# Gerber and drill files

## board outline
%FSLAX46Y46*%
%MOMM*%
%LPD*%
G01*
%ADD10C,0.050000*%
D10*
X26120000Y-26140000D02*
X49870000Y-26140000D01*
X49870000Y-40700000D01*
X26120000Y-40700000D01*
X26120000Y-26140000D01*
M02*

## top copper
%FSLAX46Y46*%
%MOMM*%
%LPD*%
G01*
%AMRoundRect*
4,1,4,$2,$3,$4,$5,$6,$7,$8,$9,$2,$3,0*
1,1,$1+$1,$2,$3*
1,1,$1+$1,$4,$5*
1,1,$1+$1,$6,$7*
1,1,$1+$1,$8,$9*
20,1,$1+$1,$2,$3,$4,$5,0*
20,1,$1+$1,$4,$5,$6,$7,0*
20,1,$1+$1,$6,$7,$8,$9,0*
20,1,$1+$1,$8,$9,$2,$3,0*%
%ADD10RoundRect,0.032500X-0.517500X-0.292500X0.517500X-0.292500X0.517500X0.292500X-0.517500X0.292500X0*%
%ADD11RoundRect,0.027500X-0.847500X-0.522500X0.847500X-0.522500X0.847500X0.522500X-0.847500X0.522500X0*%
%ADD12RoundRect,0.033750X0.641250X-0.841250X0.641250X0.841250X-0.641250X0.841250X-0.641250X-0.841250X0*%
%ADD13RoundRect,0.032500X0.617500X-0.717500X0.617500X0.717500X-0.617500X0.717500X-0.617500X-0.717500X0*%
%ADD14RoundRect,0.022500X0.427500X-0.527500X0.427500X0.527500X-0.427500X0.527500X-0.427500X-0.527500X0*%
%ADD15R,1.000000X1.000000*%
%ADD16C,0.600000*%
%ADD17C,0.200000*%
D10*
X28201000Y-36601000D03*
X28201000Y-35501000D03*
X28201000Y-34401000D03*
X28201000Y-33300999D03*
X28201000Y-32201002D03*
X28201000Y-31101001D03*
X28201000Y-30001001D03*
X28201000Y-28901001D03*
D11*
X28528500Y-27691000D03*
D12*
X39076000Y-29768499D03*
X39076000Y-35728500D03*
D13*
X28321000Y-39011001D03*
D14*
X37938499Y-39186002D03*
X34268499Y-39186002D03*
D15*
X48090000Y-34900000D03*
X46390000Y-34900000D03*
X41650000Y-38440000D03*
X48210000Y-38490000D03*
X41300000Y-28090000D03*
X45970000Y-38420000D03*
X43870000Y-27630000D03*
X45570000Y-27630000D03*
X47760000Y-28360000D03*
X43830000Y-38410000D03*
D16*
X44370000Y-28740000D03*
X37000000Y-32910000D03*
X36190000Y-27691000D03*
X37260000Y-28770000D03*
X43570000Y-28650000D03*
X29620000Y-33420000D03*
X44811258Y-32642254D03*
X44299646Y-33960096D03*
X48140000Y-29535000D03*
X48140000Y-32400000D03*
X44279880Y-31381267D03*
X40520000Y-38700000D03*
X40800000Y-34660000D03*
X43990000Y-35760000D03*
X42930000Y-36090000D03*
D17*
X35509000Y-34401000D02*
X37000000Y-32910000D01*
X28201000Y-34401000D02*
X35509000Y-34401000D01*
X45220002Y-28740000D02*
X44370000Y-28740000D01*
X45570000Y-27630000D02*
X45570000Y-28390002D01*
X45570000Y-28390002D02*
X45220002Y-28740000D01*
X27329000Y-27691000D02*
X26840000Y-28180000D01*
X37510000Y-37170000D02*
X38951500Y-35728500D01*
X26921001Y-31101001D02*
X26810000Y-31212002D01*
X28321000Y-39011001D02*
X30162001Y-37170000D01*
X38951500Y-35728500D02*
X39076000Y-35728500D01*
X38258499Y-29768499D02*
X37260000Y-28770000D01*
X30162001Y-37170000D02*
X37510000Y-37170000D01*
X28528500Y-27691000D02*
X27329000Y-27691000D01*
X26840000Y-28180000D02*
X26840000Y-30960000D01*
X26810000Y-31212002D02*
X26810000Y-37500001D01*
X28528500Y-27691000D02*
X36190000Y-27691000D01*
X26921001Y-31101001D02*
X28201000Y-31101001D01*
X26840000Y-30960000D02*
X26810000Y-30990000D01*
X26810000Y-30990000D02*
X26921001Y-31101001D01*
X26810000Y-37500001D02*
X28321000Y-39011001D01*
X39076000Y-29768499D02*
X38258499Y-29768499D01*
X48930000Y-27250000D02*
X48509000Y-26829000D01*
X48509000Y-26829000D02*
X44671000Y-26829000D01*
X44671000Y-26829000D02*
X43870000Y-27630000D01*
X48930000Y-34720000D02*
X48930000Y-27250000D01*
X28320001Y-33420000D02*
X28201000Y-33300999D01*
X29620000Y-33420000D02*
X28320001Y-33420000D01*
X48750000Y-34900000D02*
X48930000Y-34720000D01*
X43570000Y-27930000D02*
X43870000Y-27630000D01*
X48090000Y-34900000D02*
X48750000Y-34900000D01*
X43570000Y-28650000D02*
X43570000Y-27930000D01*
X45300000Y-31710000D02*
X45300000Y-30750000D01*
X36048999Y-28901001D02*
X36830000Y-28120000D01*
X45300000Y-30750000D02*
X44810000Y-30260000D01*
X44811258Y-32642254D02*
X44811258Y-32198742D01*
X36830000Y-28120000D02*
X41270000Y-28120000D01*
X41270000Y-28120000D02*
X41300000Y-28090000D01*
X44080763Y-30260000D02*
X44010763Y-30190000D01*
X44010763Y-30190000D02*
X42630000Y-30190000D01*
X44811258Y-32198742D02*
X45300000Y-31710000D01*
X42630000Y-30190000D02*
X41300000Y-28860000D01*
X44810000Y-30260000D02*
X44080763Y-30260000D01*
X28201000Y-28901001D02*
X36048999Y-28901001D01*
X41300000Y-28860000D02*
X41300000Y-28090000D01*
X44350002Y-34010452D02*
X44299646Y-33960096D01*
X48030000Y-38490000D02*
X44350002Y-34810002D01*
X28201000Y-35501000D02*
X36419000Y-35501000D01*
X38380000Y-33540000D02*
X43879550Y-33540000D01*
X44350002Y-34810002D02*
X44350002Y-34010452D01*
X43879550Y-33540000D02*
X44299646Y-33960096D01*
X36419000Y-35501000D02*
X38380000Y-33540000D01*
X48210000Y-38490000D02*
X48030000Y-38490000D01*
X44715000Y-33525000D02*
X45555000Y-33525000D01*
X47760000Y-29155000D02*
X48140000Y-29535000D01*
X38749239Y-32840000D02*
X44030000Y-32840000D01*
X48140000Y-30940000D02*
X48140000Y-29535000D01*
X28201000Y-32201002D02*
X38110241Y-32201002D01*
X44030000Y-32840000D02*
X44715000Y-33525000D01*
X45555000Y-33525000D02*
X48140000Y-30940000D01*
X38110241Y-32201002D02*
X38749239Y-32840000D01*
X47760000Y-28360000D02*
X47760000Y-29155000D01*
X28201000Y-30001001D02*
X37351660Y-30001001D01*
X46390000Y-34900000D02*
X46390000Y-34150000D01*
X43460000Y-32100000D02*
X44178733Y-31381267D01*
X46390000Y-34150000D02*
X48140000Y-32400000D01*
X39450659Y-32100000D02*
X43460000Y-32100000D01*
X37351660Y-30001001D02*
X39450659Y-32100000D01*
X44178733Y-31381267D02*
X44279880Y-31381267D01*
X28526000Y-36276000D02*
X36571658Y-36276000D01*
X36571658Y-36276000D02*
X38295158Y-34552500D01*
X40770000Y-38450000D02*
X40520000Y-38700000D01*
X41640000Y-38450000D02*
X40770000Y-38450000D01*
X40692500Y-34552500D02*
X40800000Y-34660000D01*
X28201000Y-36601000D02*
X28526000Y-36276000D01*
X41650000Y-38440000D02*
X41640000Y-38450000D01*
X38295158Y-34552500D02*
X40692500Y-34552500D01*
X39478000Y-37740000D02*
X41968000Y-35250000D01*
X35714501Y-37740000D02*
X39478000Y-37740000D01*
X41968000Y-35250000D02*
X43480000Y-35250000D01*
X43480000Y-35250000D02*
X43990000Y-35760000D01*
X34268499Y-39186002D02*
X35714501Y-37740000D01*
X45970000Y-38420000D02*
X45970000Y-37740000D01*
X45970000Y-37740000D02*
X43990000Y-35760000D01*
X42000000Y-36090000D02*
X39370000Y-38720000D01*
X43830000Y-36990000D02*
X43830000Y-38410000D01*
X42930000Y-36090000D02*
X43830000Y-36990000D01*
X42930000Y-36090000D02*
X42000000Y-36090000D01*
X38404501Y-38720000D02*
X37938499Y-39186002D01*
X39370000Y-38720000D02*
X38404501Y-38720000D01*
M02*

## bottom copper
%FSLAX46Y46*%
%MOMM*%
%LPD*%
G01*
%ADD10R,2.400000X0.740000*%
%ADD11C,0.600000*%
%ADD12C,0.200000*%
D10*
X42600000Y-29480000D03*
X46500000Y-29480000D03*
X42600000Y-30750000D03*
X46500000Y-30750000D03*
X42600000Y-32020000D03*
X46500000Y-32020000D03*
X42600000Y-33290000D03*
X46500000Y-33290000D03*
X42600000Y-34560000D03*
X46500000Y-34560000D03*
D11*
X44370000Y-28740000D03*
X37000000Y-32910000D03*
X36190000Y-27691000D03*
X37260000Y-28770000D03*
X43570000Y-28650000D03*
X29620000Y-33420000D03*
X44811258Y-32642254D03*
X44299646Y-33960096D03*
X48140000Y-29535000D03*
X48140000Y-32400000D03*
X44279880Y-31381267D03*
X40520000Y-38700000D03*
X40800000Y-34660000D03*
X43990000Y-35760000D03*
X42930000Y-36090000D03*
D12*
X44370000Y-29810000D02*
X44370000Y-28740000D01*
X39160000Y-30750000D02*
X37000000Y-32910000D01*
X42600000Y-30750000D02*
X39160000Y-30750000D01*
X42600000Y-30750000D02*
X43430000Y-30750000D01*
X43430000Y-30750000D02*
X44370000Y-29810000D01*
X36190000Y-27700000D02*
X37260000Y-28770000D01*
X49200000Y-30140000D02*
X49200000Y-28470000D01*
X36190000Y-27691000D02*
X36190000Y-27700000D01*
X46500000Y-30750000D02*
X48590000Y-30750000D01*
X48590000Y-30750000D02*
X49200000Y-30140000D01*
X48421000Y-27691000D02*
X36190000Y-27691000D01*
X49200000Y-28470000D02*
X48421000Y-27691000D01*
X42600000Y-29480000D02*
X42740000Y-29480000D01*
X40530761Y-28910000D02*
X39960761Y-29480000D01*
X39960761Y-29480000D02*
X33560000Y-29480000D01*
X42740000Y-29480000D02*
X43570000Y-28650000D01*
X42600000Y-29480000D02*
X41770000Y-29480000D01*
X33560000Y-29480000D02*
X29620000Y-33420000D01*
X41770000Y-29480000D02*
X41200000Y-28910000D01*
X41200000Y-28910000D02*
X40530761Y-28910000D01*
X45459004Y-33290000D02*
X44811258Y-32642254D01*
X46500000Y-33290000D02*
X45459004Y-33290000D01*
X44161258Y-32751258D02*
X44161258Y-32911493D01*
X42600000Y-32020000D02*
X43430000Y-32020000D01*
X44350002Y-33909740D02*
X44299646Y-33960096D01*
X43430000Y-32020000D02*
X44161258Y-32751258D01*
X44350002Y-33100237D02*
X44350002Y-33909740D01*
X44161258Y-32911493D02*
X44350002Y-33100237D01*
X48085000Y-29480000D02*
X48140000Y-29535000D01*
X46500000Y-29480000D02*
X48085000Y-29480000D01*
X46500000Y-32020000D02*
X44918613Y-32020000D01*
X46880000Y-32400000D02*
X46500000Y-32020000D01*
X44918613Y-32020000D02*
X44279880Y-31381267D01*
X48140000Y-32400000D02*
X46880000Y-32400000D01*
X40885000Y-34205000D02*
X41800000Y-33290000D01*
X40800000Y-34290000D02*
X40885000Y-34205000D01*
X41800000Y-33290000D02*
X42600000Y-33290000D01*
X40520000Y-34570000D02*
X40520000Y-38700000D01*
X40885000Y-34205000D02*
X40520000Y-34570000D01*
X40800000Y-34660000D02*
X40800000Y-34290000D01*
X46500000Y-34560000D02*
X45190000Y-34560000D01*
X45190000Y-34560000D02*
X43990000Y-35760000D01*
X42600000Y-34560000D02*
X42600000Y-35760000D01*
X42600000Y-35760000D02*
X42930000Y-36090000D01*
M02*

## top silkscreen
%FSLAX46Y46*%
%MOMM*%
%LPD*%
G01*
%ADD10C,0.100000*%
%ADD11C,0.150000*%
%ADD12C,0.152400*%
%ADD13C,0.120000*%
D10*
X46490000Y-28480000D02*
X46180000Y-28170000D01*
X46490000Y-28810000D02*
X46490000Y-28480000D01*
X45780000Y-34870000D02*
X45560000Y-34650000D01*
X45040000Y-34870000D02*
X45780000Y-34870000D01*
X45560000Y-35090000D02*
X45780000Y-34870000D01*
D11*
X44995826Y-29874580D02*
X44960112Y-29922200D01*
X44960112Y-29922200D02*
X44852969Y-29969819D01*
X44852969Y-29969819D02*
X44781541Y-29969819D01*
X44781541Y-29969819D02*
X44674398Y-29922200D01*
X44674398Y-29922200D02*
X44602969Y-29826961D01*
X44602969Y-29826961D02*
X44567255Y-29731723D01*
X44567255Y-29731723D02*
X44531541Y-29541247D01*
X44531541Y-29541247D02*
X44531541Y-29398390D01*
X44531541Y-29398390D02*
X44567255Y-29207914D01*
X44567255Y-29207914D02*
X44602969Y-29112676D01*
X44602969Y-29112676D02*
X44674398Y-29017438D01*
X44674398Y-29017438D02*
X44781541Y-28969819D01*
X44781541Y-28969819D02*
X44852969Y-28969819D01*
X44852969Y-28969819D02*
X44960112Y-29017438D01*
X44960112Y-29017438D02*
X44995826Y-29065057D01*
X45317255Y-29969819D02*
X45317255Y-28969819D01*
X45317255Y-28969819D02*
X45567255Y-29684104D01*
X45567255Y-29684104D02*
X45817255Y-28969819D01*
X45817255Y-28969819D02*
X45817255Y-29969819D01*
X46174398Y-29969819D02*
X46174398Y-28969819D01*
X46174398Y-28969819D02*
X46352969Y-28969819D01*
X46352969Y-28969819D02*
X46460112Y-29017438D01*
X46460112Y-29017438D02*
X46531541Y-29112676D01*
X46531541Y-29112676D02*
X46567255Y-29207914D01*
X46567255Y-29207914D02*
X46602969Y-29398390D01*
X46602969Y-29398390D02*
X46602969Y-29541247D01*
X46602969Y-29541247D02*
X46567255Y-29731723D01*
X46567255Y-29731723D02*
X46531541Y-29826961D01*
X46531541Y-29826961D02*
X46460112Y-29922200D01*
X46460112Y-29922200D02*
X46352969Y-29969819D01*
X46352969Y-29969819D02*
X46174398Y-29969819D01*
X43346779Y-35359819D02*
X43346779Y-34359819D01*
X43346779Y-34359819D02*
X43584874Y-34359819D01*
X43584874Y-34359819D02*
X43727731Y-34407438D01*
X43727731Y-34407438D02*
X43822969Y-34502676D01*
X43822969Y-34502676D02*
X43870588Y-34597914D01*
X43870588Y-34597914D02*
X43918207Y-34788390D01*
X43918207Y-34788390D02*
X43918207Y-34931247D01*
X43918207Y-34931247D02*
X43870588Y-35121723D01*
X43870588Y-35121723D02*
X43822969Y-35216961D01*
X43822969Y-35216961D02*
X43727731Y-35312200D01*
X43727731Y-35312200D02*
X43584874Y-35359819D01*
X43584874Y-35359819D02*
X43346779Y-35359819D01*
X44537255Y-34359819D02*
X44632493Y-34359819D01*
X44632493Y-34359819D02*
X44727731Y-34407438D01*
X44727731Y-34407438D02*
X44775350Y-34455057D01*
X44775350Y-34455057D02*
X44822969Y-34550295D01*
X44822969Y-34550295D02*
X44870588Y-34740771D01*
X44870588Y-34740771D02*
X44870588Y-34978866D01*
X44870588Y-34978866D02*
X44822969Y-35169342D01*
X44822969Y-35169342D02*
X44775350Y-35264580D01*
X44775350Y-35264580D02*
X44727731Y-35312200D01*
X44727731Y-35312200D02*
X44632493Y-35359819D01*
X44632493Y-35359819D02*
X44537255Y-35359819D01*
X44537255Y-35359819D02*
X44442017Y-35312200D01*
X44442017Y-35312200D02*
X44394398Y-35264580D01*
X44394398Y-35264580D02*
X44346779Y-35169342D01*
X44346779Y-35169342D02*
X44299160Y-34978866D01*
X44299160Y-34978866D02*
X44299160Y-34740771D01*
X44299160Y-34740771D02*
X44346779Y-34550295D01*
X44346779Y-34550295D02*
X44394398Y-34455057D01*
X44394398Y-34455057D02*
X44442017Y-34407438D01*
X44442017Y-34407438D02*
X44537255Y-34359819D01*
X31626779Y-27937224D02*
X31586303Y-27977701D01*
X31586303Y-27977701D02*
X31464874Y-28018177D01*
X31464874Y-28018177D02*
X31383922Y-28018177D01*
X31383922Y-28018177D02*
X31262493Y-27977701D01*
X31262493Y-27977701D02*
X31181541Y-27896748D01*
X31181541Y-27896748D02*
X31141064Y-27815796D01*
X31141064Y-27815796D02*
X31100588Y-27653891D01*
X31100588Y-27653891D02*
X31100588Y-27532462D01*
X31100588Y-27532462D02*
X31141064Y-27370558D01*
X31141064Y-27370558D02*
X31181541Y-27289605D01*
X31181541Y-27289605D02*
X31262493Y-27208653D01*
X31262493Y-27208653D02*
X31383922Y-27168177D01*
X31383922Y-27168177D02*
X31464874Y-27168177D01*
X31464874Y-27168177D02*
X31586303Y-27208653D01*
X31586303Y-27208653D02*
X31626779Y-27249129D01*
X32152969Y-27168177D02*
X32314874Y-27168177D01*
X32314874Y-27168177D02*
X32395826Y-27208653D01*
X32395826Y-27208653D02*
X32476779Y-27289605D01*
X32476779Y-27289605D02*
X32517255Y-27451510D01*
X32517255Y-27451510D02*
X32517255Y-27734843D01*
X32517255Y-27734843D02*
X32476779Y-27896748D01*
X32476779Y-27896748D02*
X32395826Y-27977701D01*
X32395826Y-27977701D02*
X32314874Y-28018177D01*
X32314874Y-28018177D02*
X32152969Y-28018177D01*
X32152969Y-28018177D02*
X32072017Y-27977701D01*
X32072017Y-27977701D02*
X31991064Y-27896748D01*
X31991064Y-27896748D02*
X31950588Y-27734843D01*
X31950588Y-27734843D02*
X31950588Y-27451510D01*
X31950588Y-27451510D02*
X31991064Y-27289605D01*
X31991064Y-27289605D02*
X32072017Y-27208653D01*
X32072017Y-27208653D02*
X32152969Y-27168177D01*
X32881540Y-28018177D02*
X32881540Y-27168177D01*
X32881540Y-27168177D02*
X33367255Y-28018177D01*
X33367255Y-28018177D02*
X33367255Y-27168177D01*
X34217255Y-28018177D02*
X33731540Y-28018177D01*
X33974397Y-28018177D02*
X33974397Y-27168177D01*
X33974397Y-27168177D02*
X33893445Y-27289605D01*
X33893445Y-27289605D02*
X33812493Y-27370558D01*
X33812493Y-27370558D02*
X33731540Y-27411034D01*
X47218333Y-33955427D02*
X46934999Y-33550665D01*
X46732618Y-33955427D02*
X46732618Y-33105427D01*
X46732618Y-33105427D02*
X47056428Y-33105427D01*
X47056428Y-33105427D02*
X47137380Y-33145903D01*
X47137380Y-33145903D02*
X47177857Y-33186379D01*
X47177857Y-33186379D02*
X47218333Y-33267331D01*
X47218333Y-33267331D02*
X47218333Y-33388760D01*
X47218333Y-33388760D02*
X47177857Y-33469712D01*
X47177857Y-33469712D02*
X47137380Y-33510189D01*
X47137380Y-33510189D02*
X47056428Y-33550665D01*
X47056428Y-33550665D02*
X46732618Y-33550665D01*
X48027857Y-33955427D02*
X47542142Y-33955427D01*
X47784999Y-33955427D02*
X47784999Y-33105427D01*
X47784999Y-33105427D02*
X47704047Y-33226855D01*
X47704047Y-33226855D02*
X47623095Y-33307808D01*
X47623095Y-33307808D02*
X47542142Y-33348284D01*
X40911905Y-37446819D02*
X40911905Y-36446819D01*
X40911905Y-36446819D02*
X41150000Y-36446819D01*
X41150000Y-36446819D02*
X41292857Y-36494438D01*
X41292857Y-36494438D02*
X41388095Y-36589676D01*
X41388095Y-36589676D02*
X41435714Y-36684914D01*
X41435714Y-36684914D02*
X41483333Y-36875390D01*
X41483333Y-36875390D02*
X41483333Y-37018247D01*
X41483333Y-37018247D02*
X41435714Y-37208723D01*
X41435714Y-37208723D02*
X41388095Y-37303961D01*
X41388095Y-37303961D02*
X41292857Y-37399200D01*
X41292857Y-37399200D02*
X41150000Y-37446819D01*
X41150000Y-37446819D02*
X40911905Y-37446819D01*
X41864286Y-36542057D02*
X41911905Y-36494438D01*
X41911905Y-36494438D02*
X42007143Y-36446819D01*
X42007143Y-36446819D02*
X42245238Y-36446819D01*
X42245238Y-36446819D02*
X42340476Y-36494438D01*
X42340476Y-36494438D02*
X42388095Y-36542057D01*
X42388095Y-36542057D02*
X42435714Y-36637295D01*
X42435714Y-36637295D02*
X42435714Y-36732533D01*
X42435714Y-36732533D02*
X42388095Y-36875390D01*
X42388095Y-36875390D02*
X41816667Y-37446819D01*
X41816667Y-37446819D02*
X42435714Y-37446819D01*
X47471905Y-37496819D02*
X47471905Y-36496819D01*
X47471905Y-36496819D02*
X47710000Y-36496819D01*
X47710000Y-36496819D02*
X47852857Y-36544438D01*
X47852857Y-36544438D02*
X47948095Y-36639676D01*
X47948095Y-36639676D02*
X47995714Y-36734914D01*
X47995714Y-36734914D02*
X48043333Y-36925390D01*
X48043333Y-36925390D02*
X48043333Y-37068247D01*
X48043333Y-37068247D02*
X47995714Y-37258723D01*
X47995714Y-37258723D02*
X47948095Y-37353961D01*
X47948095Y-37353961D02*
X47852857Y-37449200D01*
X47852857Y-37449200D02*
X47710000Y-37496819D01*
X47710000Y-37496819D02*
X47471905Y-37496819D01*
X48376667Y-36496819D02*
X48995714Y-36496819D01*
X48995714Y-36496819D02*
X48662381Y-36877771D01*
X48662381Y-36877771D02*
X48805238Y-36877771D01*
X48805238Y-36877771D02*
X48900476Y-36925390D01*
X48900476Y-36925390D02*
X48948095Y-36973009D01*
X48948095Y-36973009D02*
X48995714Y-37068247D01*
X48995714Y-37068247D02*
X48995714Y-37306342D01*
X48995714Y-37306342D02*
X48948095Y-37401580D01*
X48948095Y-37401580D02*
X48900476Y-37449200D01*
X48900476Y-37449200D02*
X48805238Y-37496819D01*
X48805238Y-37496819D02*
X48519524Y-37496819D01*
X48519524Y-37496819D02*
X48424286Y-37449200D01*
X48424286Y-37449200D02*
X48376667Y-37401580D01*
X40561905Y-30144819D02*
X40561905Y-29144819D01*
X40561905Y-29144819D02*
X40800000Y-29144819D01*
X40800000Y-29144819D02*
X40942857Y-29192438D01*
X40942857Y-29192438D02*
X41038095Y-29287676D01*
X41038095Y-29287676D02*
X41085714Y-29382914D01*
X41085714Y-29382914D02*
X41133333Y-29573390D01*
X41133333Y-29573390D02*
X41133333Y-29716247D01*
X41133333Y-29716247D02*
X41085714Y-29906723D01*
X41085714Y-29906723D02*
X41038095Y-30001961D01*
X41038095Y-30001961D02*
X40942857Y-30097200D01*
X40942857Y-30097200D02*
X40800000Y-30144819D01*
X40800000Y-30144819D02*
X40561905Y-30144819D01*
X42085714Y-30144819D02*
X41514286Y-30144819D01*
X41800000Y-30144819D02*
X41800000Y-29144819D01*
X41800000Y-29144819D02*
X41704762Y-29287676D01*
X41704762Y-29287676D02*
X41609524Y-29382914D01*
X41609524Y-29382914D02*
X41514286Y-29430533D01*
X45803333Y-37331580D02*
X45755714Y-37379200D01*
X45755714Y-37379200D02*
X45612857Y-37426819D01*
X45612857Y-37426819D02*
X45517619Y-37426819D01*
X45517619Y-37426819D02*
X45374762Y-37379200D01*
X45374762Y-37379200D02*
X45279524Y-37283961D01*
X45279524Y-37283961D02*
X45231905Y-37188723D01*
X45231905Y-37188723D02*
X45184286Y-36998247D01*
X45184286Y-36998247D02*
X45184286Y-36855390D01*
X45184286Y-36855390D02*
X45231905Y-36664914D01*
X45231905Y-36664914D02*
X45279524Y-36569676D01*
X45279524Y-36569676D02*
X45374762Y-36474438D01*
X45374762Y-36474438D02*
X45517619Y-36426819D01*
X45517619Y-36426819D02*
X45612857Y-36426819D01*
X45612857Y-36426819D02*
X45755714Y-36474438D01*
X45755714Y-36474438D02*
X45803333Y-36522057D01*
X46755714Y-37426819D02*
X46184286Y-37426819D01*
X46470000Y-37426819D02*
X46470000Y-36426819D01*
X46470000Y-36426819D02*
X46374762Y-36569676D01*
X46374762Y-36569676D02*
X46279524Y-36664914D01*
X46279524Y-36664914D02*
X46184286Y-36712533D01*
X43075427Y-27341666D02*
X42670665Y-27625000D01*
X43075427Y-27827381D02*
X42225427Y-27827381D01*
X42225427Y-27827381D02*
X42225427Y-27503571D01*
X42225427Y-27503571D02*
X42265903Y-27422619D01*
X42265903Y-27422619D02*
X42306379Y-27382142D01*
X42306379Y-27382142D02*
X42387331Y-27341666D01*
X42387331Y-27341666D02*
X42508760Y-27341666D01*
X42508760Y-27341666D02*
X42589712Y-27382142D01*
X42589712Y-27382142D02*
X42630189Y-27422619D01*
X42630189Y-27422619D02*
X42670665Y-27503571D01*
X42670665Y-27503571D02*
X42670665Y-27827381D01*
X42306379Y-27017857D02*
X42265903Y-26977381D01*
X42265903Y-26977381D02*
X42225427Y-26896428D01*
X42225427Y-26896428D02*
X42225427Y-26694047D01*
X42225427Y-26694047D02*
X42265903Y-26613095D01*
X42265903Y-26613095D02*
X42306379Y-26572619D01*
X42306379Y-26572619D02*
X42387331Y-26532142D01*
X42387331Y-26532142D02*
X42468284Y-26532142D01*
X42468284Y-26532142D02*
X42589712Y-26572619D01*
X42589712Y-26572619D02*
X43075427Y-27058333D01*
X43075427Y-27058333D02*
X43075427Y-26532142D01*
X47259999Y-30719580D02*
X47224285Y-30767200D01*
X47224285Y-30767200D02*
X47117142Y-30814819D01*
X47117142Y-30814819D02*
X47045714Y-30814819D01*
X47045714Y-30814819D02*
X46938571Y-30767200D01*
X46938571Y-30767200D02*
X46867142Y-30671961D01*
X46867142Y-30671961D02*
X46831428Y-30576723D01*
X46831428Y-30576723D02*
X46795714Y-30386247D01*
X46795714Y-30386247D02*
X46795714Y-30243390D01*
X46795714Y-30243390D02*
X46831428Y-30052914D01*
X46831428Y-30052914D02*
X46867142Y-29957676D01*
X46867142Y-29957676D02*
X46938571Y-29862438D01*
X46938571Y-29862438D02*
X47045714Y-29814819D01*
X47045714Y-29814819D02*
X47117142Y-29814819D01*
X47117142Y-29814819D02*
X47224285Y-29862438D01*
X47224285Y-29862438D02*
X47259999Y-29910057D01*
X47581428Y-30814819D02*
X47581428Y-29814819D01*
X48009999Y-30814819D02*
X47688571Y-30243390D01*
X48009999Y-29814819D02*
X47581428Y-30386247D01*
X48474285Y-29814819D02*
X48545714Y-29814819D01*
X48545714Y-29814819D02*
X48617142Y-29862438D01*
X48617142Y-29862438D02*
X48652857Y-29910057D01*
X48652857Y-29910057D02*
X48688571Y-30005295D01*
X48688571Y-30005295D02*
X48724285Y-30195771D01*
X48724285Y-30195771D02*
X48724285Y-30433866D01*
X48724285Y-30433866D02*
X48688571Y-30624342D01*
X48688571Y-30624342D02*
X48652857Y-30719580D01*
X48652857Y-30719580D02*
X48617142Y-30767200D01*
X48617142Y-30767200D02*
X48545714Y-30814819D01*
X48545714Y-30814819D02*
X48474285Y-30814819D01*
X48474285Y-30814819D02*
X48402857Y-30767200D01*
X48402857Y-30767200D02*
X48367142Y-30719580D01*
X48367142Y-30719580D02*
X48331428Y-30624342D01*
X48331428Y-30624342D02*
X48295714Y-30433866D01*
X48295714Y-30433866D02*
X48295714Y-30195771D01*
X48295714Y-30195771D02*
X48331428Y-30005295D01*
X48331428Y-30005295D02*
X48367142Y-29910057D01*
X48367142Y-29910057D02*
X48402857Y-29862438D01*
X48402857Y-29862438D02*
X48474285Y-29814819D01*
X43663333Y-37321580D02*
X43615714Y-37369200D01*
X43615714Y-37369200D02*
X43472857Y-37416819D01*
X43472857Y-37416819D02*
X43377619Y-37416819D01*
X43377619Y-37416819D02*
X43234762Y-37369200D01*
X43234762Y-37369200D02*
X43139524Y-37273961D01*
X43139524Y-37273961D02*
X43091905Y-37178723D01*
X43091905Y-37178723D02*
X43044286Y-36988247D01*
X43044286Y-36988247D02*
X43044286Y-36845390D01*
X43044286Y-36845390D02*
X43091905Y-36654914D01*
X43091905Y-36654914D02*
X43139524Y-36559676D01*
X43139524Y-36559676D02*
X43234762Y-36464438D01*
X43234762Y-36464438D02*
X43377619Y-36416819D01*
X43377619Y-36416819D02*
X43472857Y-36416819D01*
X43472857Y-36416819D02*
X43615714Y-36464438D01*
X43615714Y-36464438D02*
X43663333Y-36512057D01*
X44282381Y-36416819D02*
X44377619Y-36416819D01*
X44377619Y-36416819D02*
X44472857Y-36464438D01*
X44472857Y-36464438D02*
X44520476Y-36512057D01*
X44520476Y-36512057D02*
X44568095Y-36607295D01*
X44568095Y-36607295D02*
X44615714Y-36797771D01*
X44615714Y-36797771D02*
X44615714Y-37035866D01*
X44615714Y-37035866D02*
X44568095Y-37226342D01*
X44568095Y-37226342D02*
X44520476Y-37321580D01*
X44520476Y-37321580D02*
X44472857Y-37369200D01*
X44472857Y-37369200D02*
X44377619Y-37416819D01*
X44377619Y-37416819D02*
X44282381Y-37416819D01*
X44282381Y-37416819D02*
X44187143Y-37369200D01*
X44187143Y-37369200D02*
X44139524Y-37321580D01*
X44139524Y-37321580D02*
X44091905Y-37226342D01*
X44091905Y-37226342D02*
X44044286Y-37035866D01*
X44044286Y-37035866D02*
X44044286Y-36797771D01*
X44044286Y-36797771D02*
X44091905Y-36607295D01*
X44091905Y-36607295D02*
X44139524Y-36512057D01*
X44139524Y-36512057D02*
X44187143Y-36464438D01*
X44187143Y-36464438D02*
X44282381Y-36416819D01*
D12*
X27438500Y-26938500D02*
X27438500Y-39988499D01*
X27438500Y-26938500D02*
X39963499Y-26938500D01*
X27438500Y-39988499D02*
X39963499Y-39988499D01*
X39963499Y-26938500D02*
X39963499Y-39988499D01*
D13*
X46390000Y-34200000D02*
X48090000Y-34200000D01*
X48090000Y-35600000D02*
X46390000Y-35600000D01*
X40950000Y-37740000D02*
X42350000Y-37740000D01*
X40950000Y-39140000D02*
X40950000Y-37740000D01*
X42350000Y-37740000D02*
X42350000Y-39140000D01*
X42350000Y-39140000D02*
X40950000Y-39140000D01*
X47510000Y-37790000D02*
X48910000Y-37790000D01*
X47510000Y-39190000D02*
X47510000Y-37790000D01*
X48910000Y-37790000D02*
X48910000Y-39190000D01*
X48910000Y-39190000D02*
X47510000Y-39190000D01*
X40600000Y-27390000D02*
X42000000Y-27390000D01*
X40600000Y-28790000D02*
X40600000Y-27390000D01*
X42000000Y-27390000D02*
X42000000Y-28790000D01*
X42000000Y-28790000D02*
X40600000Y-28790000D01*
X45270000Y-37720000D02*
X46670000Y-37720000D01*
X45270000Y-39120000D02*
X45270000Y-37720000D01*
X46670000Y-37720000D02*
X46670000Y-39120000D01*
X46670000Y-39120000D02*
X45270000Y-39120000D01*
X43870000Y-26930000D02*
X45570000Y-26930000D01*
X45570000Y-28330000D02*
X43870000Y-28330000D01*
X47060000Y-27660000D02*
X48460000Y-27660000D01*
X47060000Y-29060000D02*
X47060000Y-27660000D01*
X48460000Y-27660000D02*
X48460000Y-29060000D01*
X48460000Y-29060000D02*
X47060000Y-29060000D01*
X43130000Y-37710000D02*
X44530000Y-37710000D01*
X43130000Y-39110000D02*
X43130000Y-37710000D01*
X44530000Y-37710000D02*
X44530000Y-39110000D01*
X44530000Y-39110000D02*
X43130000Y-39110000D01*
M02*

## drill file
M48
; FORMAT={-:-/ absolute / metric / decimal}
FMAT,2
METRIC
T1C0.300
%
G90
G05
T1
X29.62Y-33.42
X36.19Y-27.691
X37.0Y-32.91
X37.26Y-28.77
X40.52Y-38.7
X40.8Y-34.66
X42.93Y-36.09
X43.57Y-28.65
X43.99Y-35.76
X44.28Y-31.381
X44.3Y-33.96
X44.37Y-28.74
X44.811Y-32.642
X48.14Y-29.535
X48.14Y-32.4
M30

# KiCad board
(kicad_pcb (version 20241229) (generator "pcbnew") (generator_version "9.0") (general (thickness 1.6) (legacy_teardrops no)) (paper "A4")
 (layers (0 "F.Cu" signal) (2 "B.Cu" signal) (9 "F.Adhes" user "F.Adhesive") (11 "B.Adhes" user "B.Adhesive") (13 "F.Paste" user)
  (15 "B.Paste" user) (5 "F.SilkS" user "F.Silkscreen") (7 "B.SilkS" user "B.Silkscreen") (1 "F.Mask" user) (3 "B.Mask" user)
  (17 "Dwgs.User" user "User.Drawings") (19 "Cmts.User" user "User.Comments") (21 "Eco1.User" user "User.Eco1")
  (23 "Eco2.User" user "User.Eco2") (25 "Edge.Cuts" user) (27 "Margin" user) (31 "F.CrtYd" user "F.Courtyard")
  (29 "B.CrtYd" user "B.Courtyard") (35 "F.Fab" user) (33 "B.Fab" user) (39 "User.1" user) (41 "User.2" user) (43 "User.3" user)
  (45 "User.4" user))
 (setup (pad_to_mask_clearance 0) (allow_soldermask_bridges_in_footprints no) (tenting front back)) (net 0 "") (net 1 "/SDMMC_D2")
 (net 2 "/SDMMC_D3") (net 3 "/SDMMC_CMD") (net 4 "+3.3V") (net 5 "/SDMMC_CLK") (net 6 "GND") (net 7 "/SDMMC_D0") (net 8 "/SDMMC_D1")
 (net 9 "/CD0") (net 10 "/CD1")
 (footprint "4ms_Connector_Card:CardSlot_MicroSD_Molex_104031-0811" (layer "F.Cu") (at 33.6385 33.4385 -90)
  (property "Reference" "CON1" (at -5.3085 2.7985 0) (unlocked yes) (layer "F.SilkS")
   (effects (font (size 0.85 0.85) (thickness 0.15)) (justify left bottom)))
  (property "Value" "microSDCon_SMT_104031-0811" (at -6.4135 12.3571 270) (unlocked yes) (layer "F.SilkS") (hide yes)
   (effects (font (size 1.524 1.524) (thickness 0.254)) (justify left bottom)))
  (fp_line (start -6.5 6.2) (end 6.549999 6.2) (stroke (width 0.1524) (type solid)) (layer "F.SilkS"))
  (fp_line (start -6.5 6.2) (end -6.5 -6.324999) (stroke (width 0.1524) (type solid)) (layer "F.SilkS"))
  (fp_line (start 6.549999 6.2) (end 6.549999 -6.324999) (stroke (width 0.1524) (type solid)) (layer "F.SilkS"))
  (fp_line (start -6.5 -6.324999) (end 6.549999 -6.324999) (stroke (width 0.1524) (type solid)) (layer "F.SilkS"))
  (pad "1" smd roundrect (at 3.1625 5.4375) (size 1.1 0.65) (layers "F.Cu" "F.Mask" "F.Paste") (roundrect_rratio 0.05) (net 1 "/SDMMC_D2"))
  (pad "2" smd roundrect (at 2.0625 5.4375) (size 1.1 0.65) (layers "F.Cu" "F.Mask" "F.Paste") (roundrect_rratio 0.05) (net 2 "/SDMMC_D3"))
  (pad "3" smd roundrect (at 0.9625 5.4375) (size 1.1 0.65) (layers "F.Cu" "F.Mask" "F.Paste") (roundrect_rratio 0.05) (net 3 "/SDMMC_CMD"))
  (pad "4" smd roundrect (at -0.137501 5.4375) (size 1.1 0.65) (layers "F.Cu" "F.Mask" "F.Paste") (roundrect_rratio 0.05) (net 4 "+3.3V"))
  (pad "5" smd roundrect (at -1.237498 5.4375) (size 1.1 0.65) (layers "F.Cu" "F.Mask" "F.Paste") (roundrect_rratio 0.05)
   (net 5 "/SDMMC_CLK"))
  (pad "6" smd roundrect (at -2.337499 5.4375) (size 1.1 0.65) (layers "F.Cu" "F.Mask" "F.Paste") (roundrect_rratio 0.05) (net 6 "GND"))
  (pad "7" smd roundrect (at -3.437499 5.4375) (size 1.1 0.65) (layers "F.Cu" "F.Mask" "F.Paste") (roundrect_rratio 0.05)
   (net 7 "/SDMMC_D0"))
  (pad "8" smd roundrect (at -4.537499 5.4375) (size 1.1 0.65) (layers "F.Cu" "F.Mask" "F.Paste") (roundrect_rratio 0.05)
   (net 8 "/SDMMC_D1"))
  (pad "9" smd roundrect (at -5.7475 5.11) (size 1.75 1.1) (layers "F.Cu" "F.Mask" "F.Paste") (roundrect_rratio 0.025) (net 6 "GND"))
  (pad "9" smd roundrect (at -3.670001 -5.4375 90) (size 1.75 1.35) (layers "F.Cu" "F.Mask" "F.Paste") (roundrect_rratio 0.025)
   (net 6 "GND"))
  (pad "9" smd roundrect (at 2.29 -5.4375 90) (size 1.75 1.35) (layers "F.Cu" "F.Mask" "F.Paste") (roundrect_rratio 0.025) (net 6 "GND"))
  (pad "9" smd roundrect (at 5.572501 5.3175 90) (size 1.5 1.3) (layers "F.Cu" "F.Mask" "F.Paste") (roundrect_rratio 0.025) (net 6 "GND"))
  (pad "10" smd roundrect (at 5.747502 -4.299999 90) (size 1.1 0.9) (layers "F.Cu" "F.Mask" "F.Paste") (roundrect_rratio 0.025)
   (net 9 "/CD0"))
  (pad "11" smd roundrect (at 5.747502 -0.629999 90) (size 1.1 0.9) (layers "F.Cu" "F.Mask" "F.Paste") (roundrect_rratio 0.025)
   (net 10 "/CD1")))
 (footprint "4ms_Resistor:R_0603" (layer "F.Cu") (at 47.24 34.9 180)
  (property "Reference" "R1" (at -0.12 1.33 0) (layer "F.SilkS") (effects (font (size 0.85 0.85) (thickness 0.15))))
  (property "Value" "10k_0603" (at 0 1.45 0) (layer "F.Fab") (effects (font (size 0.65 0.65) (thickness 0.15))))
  (fp_line (start 0.85 0.7) (end -0.85 0.7) (stroke (width 0.12) (type solid)) (layer "F.SilkS"))
  (fp_line (start -0.85 -0.7) (end 0.85 -0.7) (stroke (width 0.12) (type solid)) (layer "F.SilkS"))
  (pad "1" smd rect (at -0.85 0 180) (size 1 1) (layers "F.Cu" "F.Mask" "F.Paste") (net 4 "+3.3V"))
  (pad "2" smd rect (at 0.85 0 180) (size 1 1) (layers "F.Cu" "F.Mask" "F.Paste") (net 7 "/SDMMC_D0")))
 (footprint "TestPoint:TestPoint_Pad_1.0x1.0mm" (layer "F.Cu") (at 41.65 38.44)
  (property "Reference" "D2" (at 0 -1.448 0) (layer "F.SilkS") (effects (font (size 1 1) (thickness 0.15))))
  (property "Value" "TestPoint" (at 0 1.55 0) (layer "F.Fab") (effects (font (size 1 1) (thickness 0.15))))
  (fp_line (start -0.7 -0.7) (end 0.7 -0.7) (stroke (width 0.12) (type solid)) (layer "F.SilkS"))
  (fp_line (start -0.7 0.7) (end -0.7 -0.7) (stroke (width 0.12) (type solid)) (layer "F.SilkS"))
  (fp_line (start 0.7 -0.7) (end 0.7 0.7) (stroke (width 0.12) (type solid)) (layer "F.SilkS"))
  (fp_line (start 0.7 0.7) (end -0.7 0.7) (stroke (width 0.12) (type solid)) (layer "F.SilkS"))
  (pad "1" smd rect (at 0 0) (size 1 1) (layers "F.Cu" "F.Mask") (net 1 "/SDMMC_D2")))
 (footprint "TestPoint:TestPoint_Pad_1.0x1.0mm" (layer "F.Cu") (at 48.21 38.49)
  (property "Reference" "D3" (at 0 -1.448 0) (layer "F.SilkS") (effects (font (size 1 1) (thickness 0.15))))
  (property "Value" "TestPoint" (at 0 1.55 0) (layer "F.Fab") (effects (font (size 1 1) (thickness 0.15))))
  (fp_line (start -0.7 -0.7) (end 0.7 -0.7) (stroke (width 0.12) (type solid)) (layer "F.SilkS"))
  (fp_line (start -0.7 0.7) (end -0.7 -0.7) (stroke (width 0.12) (type solid)) (layer "F.SilkS"))
  (fp_line (start 0.7 -0.7) (end 0.7 0.7) (stroke (width 0.12) (type solid)) (layer "F.SilkS"))
  (fp_line (start 0.7 0.7) (end -0.7 0.7) (stroke (width 0.12) (type solid)) (layer "F.SilkS"))
  (pad "1" smd rect (at 0 0) (size 1 1) (layers "F.Cu" "F.Mask") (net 2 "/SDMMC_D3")))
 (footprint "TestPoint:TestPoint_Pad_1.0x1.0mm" (layer "F.Cu") (at 41.3 28.09)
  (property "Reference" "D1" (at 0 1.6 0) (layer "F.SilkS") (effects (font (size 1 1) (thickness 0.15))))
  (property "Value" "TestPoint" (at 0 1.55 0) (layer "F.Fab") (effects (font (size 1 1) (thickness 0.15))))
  (fp_line (start -0.7 -0.7) (end 0.7 -0.7) (stroke (width 0.12) (type solid)) (layer "F.SilkS"))
  (fp_line (start -0.7 0.7) (end -0.7 -0.7) (stroke (width 0.12) (type solid)) (layer "F.SilkS"))
  (fp_line (start 0.7 -0.7) (end 0.7 0.7) (stroke (width 0.12) (type solid)) (layer "F.SilkS"))
  (fp_line (start 0.7 0.7) (end -0.7 0.7) (stroke (width 0.12) (type solid)) (layer "F.SilkS"))
  (pad "1" smd rect (at 0 0) (size 1 1) (layers "F.Cu" "F.Mask") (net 8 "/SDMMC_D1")))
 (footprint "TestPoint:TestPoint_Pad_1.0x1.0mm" (layer "F.Cu") (at 45.97 38.42)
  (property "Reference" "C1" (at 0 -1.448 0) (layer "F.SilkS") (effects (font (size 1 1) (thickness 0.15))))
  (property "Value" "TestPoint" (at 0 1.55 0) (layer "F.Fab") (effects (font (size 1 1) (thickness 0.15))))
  (fp_line (start -0.7 -0.7) (end 0.7 -0.7) (stroke (width 0.12) (type solid)) (layer "F.SilkS"))
  (fp_line (start -0.7 0.7) (end -0.7 -0.7) (stroke (width 0.12) (type solid)) (layer "F.SilkS"))
  (fp_line (start 0.7 -0.7) (end 0.7 0.7) (stroke (width 0.12) (type solid)) (layer "F.SilkS"))
  (fp_line (start 0.7 0.7) (end -0.7 0.7) (stroke (width 0.12) (type solid)) (layer "F.SilkS"))
  (pad "1" smd rect (at 0 0) (size 1 1) (layers "F.Cu" "F.Mask") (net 10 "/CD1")))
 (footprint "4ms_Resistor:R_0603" (layer "F.Cu") (at 44.72 27.63)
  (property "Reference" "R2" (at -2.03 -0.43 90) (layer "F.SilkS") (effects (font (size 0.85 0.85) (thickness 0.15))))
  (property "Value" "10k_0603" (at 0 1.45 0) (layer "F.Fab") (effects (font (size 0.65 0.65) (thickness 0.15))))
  (fp_line (start -0.85 -0.7) (end 0.85 -0.7) (stroke (width 0.12) (type solid)) (layer "F.SilkS"))
  (fp_line (start 0.85 0.7) (end -0.85 0.7) (stroke (width 0.12) (type solid)) (layer "F.SilkS"))
  (pad "1" smd rect (at -0.85 0) (size 1 1) (layers "F.Cu" "F.Mask" "F.Paste") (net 4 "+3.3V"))
  (pad "2" smd rect (at 0.85 0) (size 1 1) (layers "F.Cu" "F.Mask" "F.Paste") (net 3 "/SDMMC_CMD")))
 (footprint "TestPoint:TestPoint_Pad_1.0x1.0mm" (layer "F.Cu") (at 47.76 28.36)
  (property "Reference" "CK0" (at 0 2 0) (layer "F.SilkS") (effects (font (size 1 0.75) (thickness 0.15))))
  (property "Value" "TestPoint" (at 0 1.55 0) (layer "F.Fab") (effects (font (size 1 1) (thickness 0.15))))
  (fp_line (start -0.7 -0.7) (end 0.7 -0.7) (stroke (width 0.12) (type solid)) (layer "F.SilkS"))
  (fp_line (start -0.7 0.7) (end -0.7 -0.7) (stroke (width 0.12) (type solid)) (layer "F.SilkS"))
  (fp_line (start 0.7 -0.7) (end 0.7 0.7) (stroke (width 0.12) (type solid)) (layer "F.SilkS"))
  (fp_line (start 0.7 0.7) (end -0.7 0.7) (stroke (width 0.12) (type solid)) (layer "F.SilkS"))
  (pad "1" smd rect (at 0 0) (size 1 1) (layers "F.Cu" "F.Mask") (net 5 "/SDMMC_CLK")))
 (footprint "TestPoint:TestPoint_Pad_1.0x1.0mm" (layer "F.Cu") (at 43.83 38.41)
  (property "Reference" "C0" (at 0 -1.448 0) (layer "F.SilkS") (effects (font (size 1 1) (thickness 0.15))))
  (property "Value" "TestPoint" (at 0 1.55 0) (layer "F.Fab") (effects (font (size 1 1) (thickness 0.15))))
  (fp_line (start -0.7 -0.7) (end 0.7 -0.7) (stroke (width 0.12) (type solid)) (layer "F.SilkS"))
  (fp_line (start -0.7 0.7) (end -0.7 -0.7) (stroke (width 0.12) (type solid)) (layer "F.SilkS"))
  (fp_line (start 0.7 -0.7) (end 0.7 0.7) (stroke (width 0.12) (type solid)) (layer "F.SilkS"))
  (fp_line (start 0.7 0.7) (end -0.7 0.7) (stroke (width 0.12) (type solid)) (layer "F.SilkS"))
  (pad "1" smd rect (at 0 0) (size 1 1) (layers "F.Cu" "F.Mask") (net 9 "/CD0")))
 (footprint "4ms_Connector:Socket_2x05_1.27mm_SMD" (layer "B.Cu") (at 44.55 32.02 180)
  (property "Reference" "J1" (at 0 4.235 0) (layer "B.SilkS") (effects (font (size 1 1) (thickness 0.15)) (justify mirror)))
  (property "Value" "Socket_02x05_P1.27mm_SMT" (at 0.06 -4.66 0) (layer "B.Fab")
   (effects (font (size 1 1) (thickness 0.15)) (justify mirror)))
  (pad "1" smd rect (at 1.95 2.54 180) (size 2.4 0.74) (layers "B.Cu" "B.Mask" "B.Paste") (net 4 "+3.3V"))
  (pad "2" smd rect (at -1.95 2.54 180) (size 2.4 0.74) (layers "B.Cu" "B.Mask" "B.Paste") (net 5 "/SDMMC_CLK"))
  (pad "3" smd rect (at 1.95 1.27 180) (size 2.4 0.74) (layers "B.Cu" "B.Mask" "B.Paste") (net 3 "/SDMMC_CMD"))
  (pad "4" smd rect (at -1.95 1.27 180) (size 2.4 0.74) (layers "B.Cu" "B.Mask" "B.Paste") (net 6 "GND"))
  (pad "5" smd rect (at 1.95 0 180) (size 2.4 0.74) (layers "B.Cu" "B.Mask" "B.Paste") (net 2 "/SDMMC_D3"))
  (pad "6" smd rect (at -1.95 0 180) (size 2.4 0.74) (layers "B.Cu" "B.Mask" "B.Paste") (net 7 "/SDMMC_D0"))
  (pad "7" smd rect (at 1.95 -1.27 180) (size 2.4 0.74) (layers "B.Cu" "B.Mask" "B.Paste") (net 1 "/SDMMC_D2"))
  (pad "8" smd rect (at -1.95 -1.27 180) (size 2.4 0.74) (layers "B.Cu" "B.Mask" "B.Paste") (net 8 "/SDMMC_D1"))
  (pad "9" smd rect (at 1.95 -2.54 180) (size 2.4 0.74) (layers "B.Cu" "B.Mask" "B.Paste") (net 9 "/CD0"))
  (pad "10" smd rect (at -1.95 -2.54 180) (size 2.4 0.74) (layers "B.Cu" "B.Mask" "B.Paste") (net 10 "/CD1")))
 (gr_line (start 46.49 28.48) (end 46.18 28.17) (stroke (width 0.1) (type default)) (layer "F.SilkS"))
 (gr_line (start 46.49 28.81) (end 46.49 28.48) (stroke (width 0.1) (type default)) (layer "F.SilkS"))
 (gr_line (start 45.78 34.87) (end 45.56 34.65) (stroke (width 0.1) (type default)) (layer "F.SilkS"))
 (gr_line (start 45.04 34.87) (end 45.78 34.87) (stroke (width 0.1) (type default)) (layer "F.SilkS"))
 (gr_line (start 45.56 35.09) (end 45.78 34.87) (stroke (width 0.1) (type default)) (layer "F.SilkS"))
 (gr_rect (start 26.12 26.14) (end 49.87 40.7) (stroke (width 0.05) (type default)) (fill no) (layer "Edge.Cuts"))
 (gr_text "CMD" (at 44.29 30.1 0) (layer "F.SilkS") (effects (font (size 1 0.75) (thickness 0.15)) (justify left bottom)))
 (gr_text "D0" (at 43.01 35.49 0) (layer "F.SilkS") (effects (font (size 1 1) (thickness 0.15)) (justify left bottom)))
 (segment (start 35.509 34.401) (end 37 32.91) (width 0.2) (layer "F.Cu") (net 3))
 (segment (start 28.201 34.401) (end 35.509 34.401) (width 0.2) (layer "F.Cu") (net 3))
 (segment (start 45.220002 28.74) (end 44.37 28.74) (width 0.2) (layer "F.Cu") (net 3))
 (segment (start 45.57 27.63) (end 45.57 28.390002) (width 0.2) (layer "F.Cu") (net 3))
 (segment (start 45.57 28.390002) (end 45.220002 28.74) (width 0.2) (layer "F.Cu") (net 3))
 (via (at 44.37 28.74) (size 0.6) (drill 0.3) (layers "F.Cu" "B.Cu") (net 3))
 (via (at 37 32.91) (size 0.6) (drill 0.3) (layers "F.Cu" "B.Cu") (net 3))
 (segment (start 44.37 29.81) (end 44.37 28.74) (width 0.2) (layer "B.Cu") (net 3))
 (segment (start 39.16 30.75) (end 37 32.91) (width 0.2) (layer "B.Cu") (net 3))
 (segment (start 42.6 30.75) (end 39.16 30.75) (width 0.2) (layer "B.Cu") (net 3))
 (segment (start 42.6 30.75) (end 43.43 30.75) (width 0.2) (layer "B.Cu") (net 3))
 (segment (start 43.43 30.75) (end 44.37 29.81) (width 0.2) (layer "B.Cu") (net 3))
 (segment (start 27.329 27.691) (end 26.84 28.18) (width 0.2) (layer "F.Cu") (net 6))
 (segment (start 37.51 37.17) (end 38.9515 35.7285) (width 0.2) (layer "F.Cu") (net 6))
 (segment (start 26.921001 31.101001) (end 26.81 31.212002) (width 0.2) (layer "F.Cu") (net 6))
 (segment (start 28.321 39.011001) (end 30.162001 37.17) (width 0.2) (layer "F.Cu") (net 6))
 (segment (start 38.9515 35.7285) (end 39.076 35.7285) (width 0.2) (layer "F.Cu") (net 6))
 (segment (start 38.258499 29.768499) (end 37.26 28.77) (width 0.2) (layer "F.Cu") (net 6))
 (segment (start 30.162001 37.17) (end 37.51 37.17) (width 0.2) (layer "F.Cu") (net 6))
 (segment (start 28.5285 27.691) (end 27.329 27.691) (width 0.2) (layer "F.Cu") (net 6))
 (segment (start 26.84 28.18) (end 26.84 30.96) (width 0.2) (layer "F.Cu") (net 6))
 (segment (start 26.81 31.212002) (end 26.81 37.500001) (width 0.2) (layer "F.Cu") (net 6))
 (segment (start 28.5285 27.691) (end 36.19 27.691) (width 0.2) (layer "F.Cu") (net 6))
 (segment (start 26.921001 31.101001) (end 28.201 31.101001) (width 0.2) (layer "F.Cu") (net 6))
 (segment (start 26.84 30.96) (end 26.81 30.99) (width 0.2) (layer "F.Cu") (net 6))
 (segment (start 26.81 30.99) (end 26.921001 31.101001) (width 0.2) (layer "F.Cu") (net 6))
 (segment (start 26.81 37.500001) (end 28.321 39.011001) (width 0.2) (layer "F.Cu") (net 6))
 (segment (start 39.076 29.768499) (end 38.258499 29.768499) (width 0.2) (layer "F.Cu") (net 6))
 (via (at 36.19 27.691) (size 0.6) (drill 0.3) (layers "F.Cu" "B.Cu") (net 6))
 (via (at 37.26 28.77) (size 0.6) (drill 0.3) (layers "F.Cu" "B.Cu") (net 6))
 (segment (start 36.19 27.7) (end 37.26 28.77) (width 0.2) (layer "B.Cu") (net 6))
 (segment (start 49.2 30.14) (end 49.2 28.47) (width 0.2) (layer "B.Cu") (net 6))
 (segment (start 36.19 27.691) (end 36.19 27.7) (width 0.2) (layer "B.Cu") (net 6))
 (segment (start 46.5 30.75) (end 48.59 30.75) (width 0.2) (layer "B.Cu") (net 6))
 (segment (start 48.59 30.75) (end 49.2 30.14) (width 0.2) (layer "B.Cu") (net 6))
 (segment (start 48.421 27.691) (end 36.19 27.691) (width 0.2) (layer "B.Cu") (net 6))
 (segment (start 49.2 28.47) (end 48.421 27.691) (width 0.2) (layer "B.Cu") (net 6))
 (segment (start 48.93 27.25) (end 48.509 26.829) (width 0.2) (layer "F.Cu") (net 4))
 (segment (start 48.509 26.829) (end 44.671 26.829) (width 0.2) (layer "F.Cu") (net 4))
 (segment (start 44.671 26.829) (end 43.87 27.63) (width 0.2) (layer "F.Cu") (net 4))
 (segment (start 48.93 34.72) (end 48.93 27.25) (width 0.2) (layer "F.Cu") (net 4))
 (segment (start 28.320001 33.42) (end 28.201 33.300999) (width 0.2) (layer "F.Cu") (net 4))
 (segment (start 29.62 33.42) (end 28.320001 33.42) (width 0.2) (layer "F.Cu") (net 4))
 (segment (start 48.75 34.9) (end 48.93 34.72) (width 0.2) (layer "F.Cu") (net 4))
 (segment (start 43.57 27.93) (end 43.87 27.63) (width 0.2) (layer "F.Cu") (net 4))
 (segment (start 48.09 34.9) (end 48.75 34.9) (width 0.2) (layer "F.Cu") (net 4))
 (segment (start 43.57 28.65) (end 43.57 27.93) (width 0.2) (layer "F.Cu") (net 4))
 (via (at 43.57 28.65) (size 0.6) (drill 0.3) (layers "F.Cu" "B.Cu") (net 4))
 (via (at 29.62 33.42) (size 0.6) (drill 0.3) (layers "F.Cu" "B.Cu") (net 4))
 (segment (start 42.6 29.48) (end 42.74 29.48) (width 0.2) (layer "B.Cu") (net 4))
 (segment (start 40.530761 28.91) (end 39.960761 29.48) (width 0.2) (layer "B.Cu") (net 4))
 (segment (start 39.960761 29.48) (end 33.56 29.48) (width 0.2) (layer "B.Cu") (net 4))
 (segment (start 42.74 29.48) (end 43.57 28.65) (width 0.2) (layer "B.Cu") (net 4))
 (segment (start 42.6 29.48) (end 41.77 29.48) (width 0.2) (layer "B.Cu") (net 4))
 (segment (start 33.56 29.48) (end 29.62 33.42) (width 0.2) (layer "B.Cu") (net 4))
 (segment (start 41.77 29.48) (end 41.2 28.91) (width 0.2) (layer "B.Cu") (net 4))
 (segment (start 41.2 28.91) (end 40.530761 28.91) (width 0.2) (layer "B.Cu") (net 4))
 (segment (start 45.3 31.71) (end 45.3 30.75) (width 0.2) (layer "F.Cu") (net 8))
 (segment (start 36.048999 28.901001) (end 36.83 28.12) (width 0.2) (layer "F.Cu") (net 8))
 (segment (start 45.3 30.75) (end 44.81 30.26) (width 0.2) (layer "F.Cu") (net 8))
 (segment (start 44.811258 32.642254) (end 44.811258 32.198742) (width 0.2) (layer "F.Cu") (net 8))
 (segment (start 36.83 28.12) (end 41.27 28.12) (width 0.2) (layer "F.Cu") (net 8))
 (segment (start 41.27 28.12) (end 41.3 28.09) (width 0.2) (layer "F.Cu") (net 8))
 (segment (start 44.080763 30.26) (end 44.010763 30.19) (width 0.2) (layer "F.Cu") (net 8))
 (segment (start 44.010763 30.19) (end 42.63 30.19) (width 0.2) (layer "F.Cu") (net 8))
 (segment (start 44.811258 32.198742) (end 45.3 31.71) (width 0.2) (layer "F.Cu") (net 8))
 (segment (start 42.63 30.19) (end 41.3 28.86) (width 0.2) (layer "F.Cu") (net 8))
 (segment (start 44.81 30.26) (end 44.080763 30.26) (width 0.2) (layer "F.Cu") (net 8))
 (segment (start 28.201 28.901001) (end 36.048999 28.901001) (width 0.2) (layer "F.Cu") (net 8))
 (segment (start 41.3 28.86) (end 41.3 28.09) (width 0.2) (layer "F.Cu") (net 8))
 (via (at 44.811258 32.642254) (size 0.6) (drill 0.3) (layers "F.Cu" "B.Cu") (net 8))
 (segment (start 45.459004 33.29) (end 44.811258 32.642254) (width 0.2) (layer "B.Cu") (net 8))
 (segment (start 46.5 33.29) (end 45.459004 33.29) (width 0.2) (layer "B.Cu") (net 8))
 (segment (start 44.350002 34.010452) (end 44.299646 33.960096) (width 0.2) (layer "F.Cu") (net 2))
 (segment (start 48.03 38.49) (end 44.350002 34.810002) (width 0.2) (layer "F.Cu") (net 2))
 (segment (start 28.201 35.501) (end 36.419 35.501) (width 0.2) (layer "F.Cu") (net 2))
 (segment (start 38.38 33.54) (end 43.87955 33.54) (width 0.2) (layer "F.Cu") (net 2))
 (segment (start 44.350002 34.810002) (end 44.350002 34.010452) (width 0.2) (layer "F.Cu") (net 2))
 (segment (start 43.87955 33.54) (end 44.299646 33.960096) (width 0.2) (layer "F.Cu") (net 2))
 (segment (start 36.419 35.501) (end 38.38 33.54) (width 0.2) (layer "F.Cu") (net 2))
 (segment (start 48.21 38.49) (end 48.03 38.49) (width 0.2) (layer "F.Cu") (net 2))
 (via (at 44.299646 33.960096) (size 0.6) (drill 0.3) (layers "F.Cu" "B.Cu") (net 2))
 (segment (start 44.161258 32.751258) (end 44.161258 32.911493) (width 0.2) (layer "B.Cu") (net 2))
 (segment (start 42.6 32.02) (end 43.43 32.02) (width 0.2) (layer "B.Cu") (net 2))
 (segment (start 44.350002 33.90974) (end 44.299646 33.960096) (width 0.2) (layer "B.Cu") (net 2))
 (segment (start 43.43 32.02) (end 44.161258 32.751258) (width 0.2) (layer "B.Cu") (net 2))
 (segment (start 44.350002 33.100237) (end 44.350002 33.90974) (width 0.2) (layer "B.Cu") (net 2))
 (segment (start 44.161258 32.911493) (end 44.350002 33.100237) (width 0.2) (layer "B.Cu") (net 2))
 (segment (start 44.715 33.525) (end 45.555 33.525) (width 0.2) (layer "F.Cu") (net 5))
 (segment (start 47.76 29.155) (end 48.14 29.535) (width 0.2) (layer "F.Cu") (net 5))
 (segment (start 38.749239 32.84) (end 44.03 32.84) (width 0.2) (layer "F.Cu") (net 5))
 (segment (start 48.14 30.94) (end 48.14 29.535) (width 0.2) (layer "F.Cu") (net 5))
 (segment (start 28.201 32.201002) (end 38.110241 32.201002) (width 0.2) (layer "F.Cu") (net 5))
 (segment (start 44.03 32.84) (end 44.715 33.525) (width 0.2) (layer "F.Cu") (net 5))
 (segment (start 45.555 33.525) (end 48.14 30.94) (width 0.2) (layer "F.Cu") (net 5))
 (segment (start 38.110241 32.201002) (end 38.749239 32.84) (width 0.2) (layer "F.Cu") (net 5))
 (segment (start 47.76 28.36) (end 47.76 29.155) (width 0.2) (layer "F.Cu") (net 5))
 (via (at 48.14 29.535) (size 0.6) (drill 0.3) (layers "F.Cu" "B.Cu") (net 5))
 (segment (start 48.085 29.48) (end 48.14 29.535) (width 0.2) (layer "B.Cu") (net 5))
 (segment (start 46.5 29.48) (end 48.085 29.48) (width 0.2) (layer "B.Cu") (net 5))
 (segment (start 28.201 30.001001) (end 37.35166 30.001001) (width 0.2) (layer "F.Cu") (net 7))
 (segment (start 46.39 34.9) (end 46.39 34.15) (width 0.2) (layer "F.Cu") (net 7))
 (segment (start 43.46 32.1) (end 44.178733 31.381267) (width 0.2) (layer "F.Cu") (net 7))
 (segment (start 46.39 34.15) (end 48.14 32.4) (width 0.2) (layer "F.Cu") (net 7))
 (segment (start 39.450659 32.1) (end 43.46 32.1) (width 0.2) (layer "F.Cu") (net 7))
 (segment (start 37.35166 30.001001) (end 39.450659 32.1) (width 0.2) (layer "F.Cu") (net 7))
 (segment (start 44.178733 31.381267) (end 44.27988 31.381267) (width 0.2) (layer "F.Cu") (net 7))
 (via (at 48.14 32.4) (size 0.6) (drill 0.3) (layers "F.Cu" "B.Cu") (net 7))
 (via (at 44.27988 31.381267) (size 0.6) (drill 0.3) (layers "F.Cu" "B.Cu") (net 7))
 (segment (start 46.5 32.02) (end 44.918613 32.02) (width 0.2) (layer "B.Cu") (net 7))
 (segment (start 46.88 32.4) (end 46.5 32.02) (width 0.2) (layer "B.Cu") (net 7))
 (segment (start 44.918613 32.02) (end 44.27988 31.381267) (width 0.2) (layer "B.Cu") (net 7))
 (segment (start 48.14 32.4) (end 46.88 32.4) (width 0.2) (layer "B.Cu") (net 7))
 (segment (start 28.526 36.276) (end 36.571658 36.276) (width 0.2) (layer "F.Cu") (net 1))
 (segment (start 36.571658 36.276) (end 38.295158 34.5525) (width 0.2) (layer "F.Cu") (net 1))
 (segment (start 40.77 38.45) (end 40.52 38.7) (width 0.2) (layer "F.Cu") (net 1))
 (segment (start 41.64 38.45) (end 40.77 38.45) (width 0.2) (layer "F.Cu") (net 1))
 (segment (start 40.6925 34.5525) (end 40.8 34.66) (width 0.2) (layer "F.Cu") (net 1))
 (segment (start 28.201 36.601) (end 28.526 36.276) (width 0.2) (layer "F.Cu") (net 1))
 (segment (start 41.65 38.44) (end 41.64 38.45) (width 0.2) (layer "F.Cu") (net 1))
 (segment (start 38.295158 34.5525) (end 40.6925 34.5525) (width 0.2) (layer "F.Cu") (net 1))
 (via (at 40.52 38.7) (size 0.6) (drill 0.3) (layers "F.Cu" "B.Cu") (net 1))
 (via (at 40.8 34.66) (size 0.6) (drill 0.3) (layers "F.Cu" "B.Cu") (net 1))
 (segment (start 40.885 34.205) (end 41.8 33.29) (width 0.2) (layer "B.Cu") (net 1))
 (segment (start 40.8 34.29) (end 40.885 34.205) (width 0.2) (layer "B.Cu") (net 1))
 (segment (start 41.8 33.29) (end 42.6 33.29) (width 0.2) (layer "B.Cu") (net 1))
 (segment (start 40.52 34.57) (end 40.52 38.7) (width 0.2) (layer "B.Cu") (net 1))
 (segment (start 40.885 34.205) (end 40.52 34.57) (width 0.2) (layer "B.Cu") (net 1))
 (segment (start 40.8 34.66) (end 40.8 34.29) (width 0.2) (layer "B.Cu") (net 1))
 (segment (start 39.478 37.74) (end 41.968 35.25) (width 0.2) (layer "F.Cu") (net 10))
 (segment (start 35.714501 37.74) (end 39.478 37.74) (width 0.2) (layer "F.Cu") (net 10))
 (segment (start 41.968 35.25) (end 43.48 35.25) (width 0.2) (layer "F.Cu") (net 10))
 (segment (start 43.48 35.25) (end 43.99 35.76) (width 0.2) (layer "F.Cu") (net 10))
 (segment (start 34.268499 39.186002) (end 35.714501 37.74) (width 0.2) (layer "F.Cu") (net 10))
 (segment (start 45.97 38.42) (end 45.97 37.74) (width 0.2) (layer "F.Cu") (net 10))
 (segment (start 45.97 37.74) (end 43.99 35.76) (width 0.2) (layer "F.Cu") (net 10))
 (via (at 43.99 35.76) (size 0.6) (drill 0.3) (layers "F.Cu" "B.Cu") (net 10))
 (segment (start 46.5 34.56) (end 45.19 34.56) (width 0.2) (layer "B.Cu") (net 10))
 (segment (start 45.19 34.56) (end 43.99 35.76) (width 0.2) (layer "B.Cu") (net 10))
 (segment (start 42 36.09) (end 39.37 38.72) (width 0.2) (layer "F.Cu") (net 9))
 (segment (start 43.83 36.99) (end 43.83 38.41) (width 0.2) (layer "F.Cu") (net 9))
 (segment (start 42.93 36.09) (end 43.83 36.99) (width 0.2) (layer "F.Cu") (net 9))
 (segment (start 42.93 36.09) (end 42 36.09) (width 0.2) (layer "F.Cu") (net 9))
 (segment (start 38.404501 38.72) (end 37.938499 39.186002) (width 0.2) (layer "F.Cu") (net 9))
 (segment (start 39.37 38.72) (end 38.404501 38.72) (width 0.2) (layer "F.Cu") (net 9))
 (via (at 42.93 36.09) (size 0.6) (drill 0.3) (layers "F.Cu" "B.Cu") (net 9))
 (segment (start 42.6 34.56) (end 42.6 35.76) (width 0.2) (layer "B.Cu") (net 9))
 (segment (start 42.6 35.76) (end 42.93 36.09) (width 0.2) (layer "B.Cu") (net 9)))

